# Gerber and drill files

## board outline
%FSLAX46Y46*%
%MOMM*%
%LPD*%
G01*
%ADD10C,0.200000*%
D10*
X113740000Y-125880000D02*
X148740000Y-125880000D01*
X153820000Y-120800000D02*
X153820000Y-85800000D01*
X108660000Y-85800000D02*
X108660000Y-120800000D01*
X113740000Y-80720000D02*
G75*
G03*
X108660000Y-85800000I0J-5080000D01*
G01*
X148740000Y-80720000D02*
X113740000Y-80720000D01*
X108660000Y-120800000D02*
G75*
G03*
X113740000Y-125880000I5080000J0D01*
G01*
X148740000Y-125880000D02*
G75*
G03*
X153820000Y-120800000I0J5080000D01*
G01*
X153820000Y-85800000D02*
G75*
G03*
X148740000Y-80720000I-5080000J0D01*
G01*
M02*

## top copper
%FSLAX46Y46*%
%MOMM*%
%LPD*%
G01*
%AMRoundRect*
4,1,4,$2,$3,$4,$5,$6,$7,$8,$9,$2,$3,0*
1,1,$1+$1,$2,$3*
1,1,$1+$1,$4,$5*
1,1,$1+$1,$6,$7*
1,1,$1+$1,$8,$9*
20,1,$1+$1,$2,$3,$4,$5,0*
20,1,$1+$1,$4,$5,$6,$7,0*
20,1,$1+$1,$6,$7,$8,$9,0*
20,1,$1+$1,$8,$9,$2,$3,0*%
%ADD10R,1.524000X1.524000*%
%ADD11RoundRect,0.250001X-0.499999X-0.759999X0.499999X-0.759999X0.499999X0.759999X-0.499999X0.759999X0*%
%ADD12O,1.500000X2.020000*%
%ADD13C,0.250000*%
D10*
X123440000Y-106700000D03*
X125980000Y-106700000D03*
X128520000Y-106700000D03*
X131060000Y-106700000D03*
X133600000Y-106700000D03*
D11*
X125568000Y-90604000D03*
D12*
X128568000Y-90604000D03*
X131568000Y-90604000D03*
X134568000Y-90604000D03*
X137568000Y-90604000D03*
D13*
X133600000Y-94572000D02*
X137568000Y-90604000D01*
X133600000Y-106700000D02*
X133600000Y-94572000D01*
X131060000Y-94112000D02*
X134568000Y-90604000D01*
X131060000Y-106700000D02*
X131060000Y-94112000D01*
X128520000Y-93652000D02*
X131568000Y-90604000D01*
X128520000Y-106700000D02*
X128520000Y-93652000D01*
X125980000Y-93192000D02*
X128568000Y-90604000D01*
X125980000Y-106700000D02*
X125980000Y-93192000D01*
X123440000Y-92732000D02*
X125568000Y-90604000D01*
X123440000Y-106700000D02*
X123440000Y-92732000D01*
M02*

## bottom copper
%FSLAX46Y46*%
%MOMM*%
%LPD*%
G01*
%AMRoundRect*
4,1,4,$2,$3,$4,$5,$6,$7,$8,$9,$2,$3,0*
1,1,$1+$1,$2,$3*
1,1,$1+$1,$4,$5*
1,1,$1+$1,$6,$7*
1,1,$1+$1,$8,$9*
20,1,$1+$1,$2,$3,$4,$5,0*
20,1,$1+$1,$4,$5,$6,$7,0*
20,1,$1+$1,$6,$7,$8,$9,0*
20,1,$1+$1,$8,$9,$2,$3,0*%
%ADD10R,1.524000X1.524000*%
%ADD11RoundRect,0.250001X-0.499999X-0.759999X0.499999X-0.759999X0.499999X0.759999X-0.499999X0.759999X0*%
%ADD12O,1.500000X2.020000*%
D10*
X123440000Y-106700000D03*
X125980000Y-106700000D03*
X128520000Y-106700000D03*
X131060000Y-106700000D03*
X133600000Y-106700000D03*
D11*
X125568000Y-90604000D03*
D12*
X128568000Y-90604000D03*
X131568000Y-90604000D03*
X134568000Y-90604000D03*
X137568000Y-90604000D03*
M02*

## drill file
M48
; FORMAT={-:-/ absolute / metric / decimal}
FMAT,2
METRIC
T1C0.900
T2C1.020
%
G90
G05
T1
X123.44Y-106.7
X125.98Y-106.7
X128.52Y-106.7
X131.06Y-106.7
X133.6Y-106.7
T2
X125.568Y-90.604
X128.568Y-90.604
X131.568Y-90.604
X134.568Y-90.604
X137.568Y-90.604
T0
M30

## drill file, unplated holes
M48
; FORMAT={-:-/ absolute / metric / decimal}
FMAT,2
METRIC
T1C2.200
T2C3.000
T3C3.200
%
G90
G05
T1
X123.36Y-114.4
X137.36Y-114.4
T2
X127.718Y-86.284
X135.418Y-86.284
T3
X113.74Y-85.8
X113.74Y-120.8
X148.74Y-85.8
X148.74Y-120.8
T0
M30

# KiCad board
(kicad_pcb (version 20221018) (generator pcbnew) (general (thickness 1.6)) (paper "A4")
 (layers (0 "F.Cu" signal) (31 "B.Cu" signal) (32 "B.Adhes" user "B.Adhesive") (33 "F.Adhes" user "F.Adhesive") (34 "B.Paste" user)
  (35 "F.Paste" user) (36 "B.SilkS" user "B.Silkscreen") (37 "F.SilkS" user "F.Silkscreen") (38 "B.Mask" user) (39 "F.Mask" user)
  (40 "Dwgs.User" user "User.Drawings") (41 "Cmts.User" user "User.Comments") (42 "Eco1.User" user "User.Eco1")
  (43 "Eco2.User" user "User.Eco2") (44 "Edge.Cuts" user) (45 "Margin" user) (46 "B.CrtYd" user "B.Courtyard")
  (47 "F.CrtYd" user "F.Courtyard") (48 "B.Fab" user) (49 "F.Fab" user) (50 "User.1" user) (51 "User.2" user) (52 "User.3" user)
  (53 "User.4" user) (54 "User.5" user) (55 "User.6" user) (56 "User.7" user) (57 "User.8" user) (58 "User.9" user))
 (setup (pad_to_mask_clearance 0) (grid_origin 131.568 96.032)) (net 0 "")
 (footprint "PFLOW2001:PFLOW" (layer "F.Cu") (at 141.22 103.5 180)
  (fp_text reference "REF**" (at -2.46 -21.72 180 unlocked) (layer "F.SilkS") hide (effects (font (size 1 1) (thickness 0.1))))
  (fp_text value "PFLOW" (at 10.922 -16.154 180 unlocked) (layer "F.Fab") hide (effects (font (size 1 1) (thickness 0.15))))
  (pad "" np_thru_hole circle (at 3.86 -10.9 180) (size 2.2 2.2) (drill 2.2) (layers "F&B.Cu" "*.Mask"))
  (pad "" np_thru_hole circle (at 17.86 -10.9 180) (size 2.2 2.2) (drill 2.2) (layers "F&B.Cu" "*.Mask"))
  (pad "1" thru_hole rect (at 7.62 -3.2 180) (size 1.524 1.524) (drill 0.9) (layers "*.Cu" "*.Mask"))
  (pad "2" thru_hole rect (at 10.16 -3.2 180) (size 1.524 1.524) (drill 0.9) (layers "*.Cu" "*.Mask"))
  (pad "3" thru_hole rect (at 12.7 -3.2 180) (size 1.524 1.524) (drill 0.9) (layers "*.Cu" "*.Mask"))
  (pad "4" thru_hole rect (at 15.24 -3.2 180) (size 1.524 1.524) (drill 0.9) (layers "*.Cu" "*.Mask"))
  (pad "5" thru_hole rect (at 17.78 -3.2 180) (size 1.524 1.524) (drill 0.9) (layers "*.Cu" "*.Mask")))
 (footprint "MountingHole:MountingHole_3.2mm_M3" (layer "F.Cu") (at 113.74 120.8)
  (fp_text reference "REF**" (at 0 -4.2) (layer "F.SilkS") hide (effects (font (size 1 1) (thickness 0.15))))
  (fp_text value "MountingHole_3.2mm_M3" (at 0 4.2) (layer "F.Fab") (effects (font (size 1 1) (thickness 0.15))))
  (pad "" np_thru_hole circle (at 0 0) (size 3.2 3.2) (drill 3.2) (layers "F&B.Cu" "*.Mask")))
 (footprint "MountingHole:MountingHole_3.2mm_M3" (layer "F.Cu") (at 148.74 120.8)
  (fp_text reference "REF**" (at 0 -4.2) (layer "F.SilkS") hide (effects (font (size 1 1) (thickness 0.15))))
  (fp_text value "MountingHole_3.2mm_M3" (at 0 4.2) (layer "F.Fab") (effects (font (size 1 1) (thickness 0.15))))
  (pad "" np_thru_hole circle (at 0 0) (size 3.2 3.2) (drill 3.2) (layers "*.Cu" "*.Mask")))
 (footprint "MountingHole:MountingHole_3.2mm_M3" (layer "F.Cu") (at 113.74 85.8)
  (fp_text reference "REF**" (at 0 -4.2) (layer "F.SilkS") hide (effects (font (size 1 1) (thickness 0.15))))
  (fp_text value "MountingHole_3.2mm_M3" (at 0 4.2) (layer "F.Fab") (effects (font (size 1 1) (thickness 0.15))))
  (pad "" np_thru_hole circle (at 0 0) (size 3.2 3.2) (drill 3.2) (layers "*.Cu" "*.Mask")))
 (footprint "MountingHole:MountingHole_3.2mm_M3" (layer "F.Cu") (at 148.74 85.8)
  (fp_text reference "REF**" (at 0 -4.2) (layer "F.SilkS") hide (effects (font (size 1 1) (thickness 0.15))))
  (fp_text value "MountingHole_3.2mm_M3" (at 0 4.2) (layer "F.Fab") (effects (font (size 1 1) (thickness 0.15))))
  (pad "" np_thru_hole circle (at 0 0) (size 3.2 3.2) (drill 3.2) (layers "F&B.Cu" "*.Mask")))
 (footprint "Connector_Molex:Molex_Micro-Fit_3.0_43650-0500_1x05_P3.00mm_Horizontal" (layer "F.Cu") (at 125.568 90.604)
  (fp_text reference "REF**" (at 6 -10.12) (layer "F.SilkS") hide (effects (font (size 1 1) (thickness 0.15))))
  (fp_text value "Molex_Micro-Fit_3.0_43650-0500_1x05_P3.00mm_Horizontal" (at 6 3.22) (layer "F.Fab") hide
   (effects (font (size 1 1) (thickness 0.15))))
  (pad "" np_thru_hole circle (at 2.15 -4.32) (size 3 3) (drill 3) (layers "*.Cu" "*.Mask"))
  (pad "" np_thru_hole circle (at 9.85 -4.32) (size 3 3) (drill 3) (layers "*.Cu" "*.Mask"))
  (pad "1" thru_hole roundrect (at 0 0) (size 1.5 2.02) (drill 1.02) (layers "*.Cu" "*.Mask") (roundrect_rratio 0.1666673333))
  (pad "2" thru_hole oval (at 3 0) (size 1.5 2.02) (drill 1.02) (layers "*.Cu" "*.Mask"))
  (pad "3" thru_hole oval (at 6 0) (size 1.5 2.02) (drill 1.02) (layers "*.Cu" "*.Mask"))
  (pad "4" thru_hole oval (at 9 0) (size 1.5 2.02) (drill 1.02) (layers "*.Cu" "*.Mask"))
  (pad "5" thru_hole oval (at 12 0) (size 1.5 2.02) (drill 1.02) (layers "*.Cu" "*.Mask")))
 (gr_line (start 113.74 125.88) (end 148.74 125.88) (stroke (width 0.2) (type default)) (layer "Edge.Cuts"))
 (gr_line (start 153.82 120.8) (end 153.82 85.8) (stroke (width 0.2) (type default)) (layer "Edge.Cuts"))
 (gr_line (start 108.66 85.8) (end 108.66 120.8) (stroke (width 0.2) (type default)) (layer "Edge.Cuts"))
 (gr_arc (start 108.66 85.8) (mid 110.147898 82.207898) (end 113.74 80.72) (stroke (width 0.2) (type default)) (layer "Edge.Cuts"))
 (gr_line (start 148.74 80.72) (end 113.74 80.72) (stroke (width 0.2) (type default)) (layer "Edge.Cuts"))
 (gr_arc (start 113.74 125.88) (mid 110.147898 124.392102) (end 108.66 120.8) (stroke (width 0.2) (type default)) (layer "Edge.Cuts"))
 (gr_arc (start 153.82 120.8) (mid 152.332102 124.392102) (end 148.74 125.88) (stroke (width 0.2) (type default)) (layer "Edge.Cuts"))
 (gr_arc (start 148.74 80.72) (mid 152.332102 82.207898) (end 153.82 85.8) (stroke (width 0.2) (type default)) (layer "Edge.Cuts"))
 (segment (start 123.44 106.7) (end 123.44 92.732) (width 0.25) (layer "F.Cu") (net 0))
 (segment (start 131.06 94.112) (end 134.568 90.604) (width 0.25) (layer "F.Cu") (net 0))
 (segment (start 133.6 94.572) (end 137.568 90.604) (width 0.25) (layer "F.Cu") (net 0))
 (segment (start 128.52 93.652) (end 131.568 90.604) (width 0.25) (layer "F.Cu") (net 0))
 (segment (start 125.98 93.192) (end 128.568 90.604) (width 0.25) (layer "F.Cu") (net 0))
 (segment (start 131.06 106.7) (end 131.06 94.112) (width 0.25) (layer "F.Cu") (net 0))
 (segment (start 125.98 106.7) (end 125.98 93.192) (width 0.25) (layer "F.Cu") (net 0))
 (segment (start 133.6 106.7) (end 133.6 94.572) (width 0.25) (layer "F.Cu") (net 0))
 (segment (start 128.52 106.7) (end 128.52 93.652) (width 0.25) (layer "F.Cu") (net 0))
 (segment (start 123.44 92.732) (end 125.568 90.604) (width 0.25) (layer "F.Cu") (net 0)))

